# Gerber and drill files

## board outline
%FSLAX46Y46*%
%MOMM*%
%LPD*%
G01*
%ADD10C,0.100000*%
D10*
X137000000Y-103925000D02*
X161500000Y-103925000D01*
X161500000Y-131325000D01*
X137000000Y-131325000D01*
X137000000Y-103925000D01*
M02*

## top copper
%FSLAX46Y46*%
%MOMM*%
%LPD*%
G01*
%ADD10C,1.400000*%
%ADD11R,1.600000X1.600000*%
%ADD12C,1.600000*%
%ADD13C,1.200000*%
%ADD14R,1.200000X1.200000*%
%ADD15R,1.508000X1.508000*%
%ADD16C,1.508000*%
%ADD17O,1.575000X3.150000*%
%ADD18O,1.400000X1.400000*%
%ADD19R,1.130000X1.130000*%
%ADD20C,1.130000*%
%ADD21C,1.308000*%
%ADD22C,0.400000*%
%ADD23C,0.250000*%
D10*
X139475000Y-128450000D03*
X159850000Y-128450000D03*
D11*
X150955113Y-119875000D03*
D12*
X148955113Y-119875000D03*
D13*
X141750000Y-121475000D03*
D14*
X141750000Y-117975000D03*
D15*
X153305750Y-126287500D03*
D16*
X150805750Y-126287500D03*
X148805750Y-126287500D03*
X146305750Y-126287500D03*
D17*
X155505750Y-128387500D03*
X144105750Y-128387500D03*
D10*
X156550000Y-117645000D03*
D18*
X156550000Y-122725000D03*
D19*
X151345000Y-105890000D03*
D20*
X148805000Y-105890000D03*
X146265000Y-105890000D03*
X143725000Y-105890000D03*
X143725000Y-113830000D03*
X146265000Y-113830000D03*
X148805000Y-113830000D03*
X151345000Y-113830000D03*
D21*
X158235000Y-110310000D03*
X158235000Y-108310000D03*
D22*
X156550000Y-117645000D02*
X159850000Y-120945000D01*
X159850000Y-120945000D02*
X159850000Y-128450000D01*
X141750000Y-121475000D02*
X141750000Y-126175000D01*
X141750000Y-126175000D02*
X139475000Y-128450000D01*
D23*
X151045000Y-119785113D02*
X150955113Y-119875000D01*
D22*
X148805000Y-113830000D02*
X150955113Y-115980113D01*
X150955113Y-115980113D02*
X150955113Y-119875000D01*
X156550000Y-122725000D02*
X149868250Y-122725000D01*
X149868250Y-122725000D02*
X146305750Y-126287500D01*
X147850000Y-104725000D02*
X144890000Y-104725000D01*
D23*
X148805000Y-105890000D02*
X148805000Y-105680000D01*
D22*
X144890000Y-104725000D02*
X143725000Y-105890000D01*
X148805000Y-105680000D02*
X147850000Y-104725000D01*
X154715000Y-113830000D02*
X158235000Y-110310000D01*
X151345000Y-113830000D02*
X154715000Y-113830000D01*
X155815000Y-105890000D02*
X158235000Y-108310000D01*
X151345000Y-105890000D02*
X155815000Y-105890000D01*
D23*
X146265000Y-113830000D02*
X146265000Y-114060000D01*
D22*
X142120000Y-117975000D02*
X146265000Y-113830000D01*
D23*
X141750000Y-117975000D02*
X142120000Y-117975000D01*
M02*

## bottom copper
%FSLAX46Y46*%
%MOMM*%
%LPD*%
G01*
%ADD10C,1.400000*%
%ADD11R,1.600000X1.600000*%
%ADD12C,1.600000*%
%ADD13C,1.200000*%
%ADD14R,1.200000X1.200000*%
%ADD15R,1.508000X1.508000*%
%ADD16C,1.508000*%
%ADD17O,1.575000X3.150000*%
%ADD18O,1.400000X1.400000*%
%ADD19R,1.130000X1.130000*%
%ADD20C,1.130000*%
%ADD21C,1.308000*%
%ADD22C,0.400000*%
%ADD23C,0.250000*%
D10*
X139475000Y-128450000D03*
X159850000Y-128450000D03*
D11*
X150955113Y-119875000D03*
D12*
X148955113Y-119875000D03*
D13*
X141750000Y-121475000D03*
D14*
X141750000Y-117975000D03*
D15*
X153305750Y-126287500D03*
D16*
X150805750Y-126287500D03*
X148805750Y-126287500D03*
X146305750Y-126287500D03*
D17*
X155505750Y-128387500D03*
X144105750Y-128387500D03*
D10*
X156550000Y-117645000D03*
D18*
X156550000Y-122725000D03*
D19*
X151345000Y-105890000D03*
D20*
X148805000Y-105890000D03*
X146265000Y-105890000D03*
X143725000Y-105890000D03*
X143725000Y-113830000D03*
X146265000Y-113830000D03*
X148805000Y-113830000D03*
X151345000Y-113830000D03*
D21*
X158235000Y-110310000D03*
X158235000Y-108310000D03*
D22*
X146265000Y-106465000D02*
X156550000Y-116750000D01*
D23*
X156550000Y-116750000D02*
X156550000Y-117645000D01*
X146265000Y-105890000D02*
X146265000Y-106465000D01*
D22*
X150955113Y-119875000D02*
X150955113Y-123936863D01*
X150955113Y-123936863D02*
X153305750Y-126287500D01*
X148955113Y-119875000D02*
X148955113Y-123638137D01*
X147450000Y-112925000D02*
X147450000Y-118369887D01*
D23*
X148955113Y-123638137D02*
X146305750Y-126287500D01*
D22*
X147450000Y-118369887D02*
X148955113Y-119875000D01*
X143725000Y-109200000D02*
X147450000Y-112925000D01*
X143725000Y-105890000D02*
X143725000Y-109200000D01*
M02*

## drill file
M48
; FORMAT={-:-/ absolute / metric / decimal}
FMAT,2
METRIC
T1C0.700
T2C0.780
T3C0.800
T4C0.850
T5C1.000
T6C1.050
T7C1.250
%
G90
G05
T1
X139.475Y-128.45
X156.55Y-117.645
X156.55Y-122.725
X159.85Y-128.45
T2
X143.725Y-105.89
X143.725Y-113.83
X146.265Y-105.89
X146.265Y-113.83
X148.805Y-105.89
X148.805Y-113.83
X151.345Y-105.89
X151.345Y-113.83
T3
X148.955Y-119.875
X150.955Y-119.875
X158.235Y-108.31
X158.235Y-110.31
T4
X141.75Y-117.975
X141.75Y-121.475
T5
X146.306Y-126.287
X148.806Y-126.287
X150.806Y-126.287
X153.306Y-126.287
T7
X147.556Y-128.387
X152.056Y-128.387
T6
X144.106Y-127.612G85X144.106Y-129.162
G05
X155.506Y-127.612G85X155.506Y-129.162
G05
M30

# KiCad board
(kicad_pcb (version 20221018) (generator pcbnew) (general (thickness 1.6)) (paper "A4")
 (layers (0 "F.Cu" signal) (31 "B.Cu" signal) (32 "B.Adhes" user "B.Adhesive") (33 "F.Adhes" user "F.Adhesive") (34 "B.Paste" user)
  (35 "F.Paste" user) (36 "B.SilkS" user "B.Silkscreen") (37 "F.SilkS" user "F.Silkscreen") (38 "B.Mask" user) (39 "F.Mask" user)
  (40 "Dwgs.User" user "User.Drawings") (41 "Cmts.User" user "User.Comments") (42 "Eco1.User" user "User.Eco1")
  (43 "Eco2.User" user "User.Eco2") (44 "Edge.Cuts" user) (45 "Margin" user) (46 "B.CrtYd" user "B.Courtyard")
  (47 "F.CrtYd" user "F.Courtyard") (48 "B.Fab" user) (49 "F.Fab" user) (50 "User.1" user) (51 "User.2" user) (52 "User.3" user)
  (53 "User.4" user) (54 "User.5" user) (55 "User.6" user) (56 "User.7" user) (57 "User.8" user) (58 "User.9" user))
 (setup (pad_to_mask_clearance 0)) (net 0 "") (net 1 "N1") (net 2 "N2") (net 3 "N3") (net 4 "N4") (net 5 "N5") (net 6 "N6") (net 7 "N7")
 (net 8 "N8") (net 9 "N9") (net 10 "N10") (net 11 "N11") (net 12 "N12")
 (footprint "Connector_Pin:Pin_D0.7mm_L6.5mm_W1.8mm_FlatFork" (layer "F.Cu") (at 139.475 128.45)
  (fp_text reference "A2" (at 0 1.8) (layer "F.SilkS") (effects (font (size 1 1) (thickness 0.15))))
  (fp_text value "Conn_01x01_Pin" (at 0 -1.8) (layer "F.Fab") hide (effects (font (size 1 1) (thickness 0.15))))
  (pad "1" thru_hole circle (at 0 0) (size 1.4 1.4) (drill 0.7) (layers "*.Cu" "*.Mask") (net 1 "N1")))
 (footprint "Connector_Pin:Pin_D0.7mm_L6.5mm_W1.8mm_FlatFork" (layer "F.Cu") (at 159.85 128.45)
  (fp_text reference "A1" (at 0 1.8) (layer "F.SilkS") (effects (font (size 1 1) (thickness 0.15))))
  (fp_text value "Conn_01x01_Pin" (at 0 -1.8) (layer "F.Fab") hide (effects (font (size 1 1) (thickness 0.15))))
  (pad "1" thru_hole circle (at 0 0) (size 1.4 1.4) (drill 0.7) (layers "*.Cu" "*.Mask") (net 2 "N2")))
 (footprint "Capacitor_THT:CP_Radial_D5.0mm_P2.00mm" (layer "F.Cu") (at 150.955113 119.875 180)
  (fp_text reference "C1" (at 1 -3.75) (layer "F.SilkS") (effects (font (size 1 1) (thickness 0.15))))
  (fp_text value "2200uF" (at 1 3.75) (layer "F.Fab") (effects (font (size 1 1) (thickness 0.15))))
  (pad "1" thru_hole rect (at 0 0 180) (size 1.6 1.6) (drill 0.8) (layers "*.Cu" "*.Mask") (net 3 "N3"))
  (pad "2" thru_hole circle (at 2 0 180) (size 1.6 1.6) (drill 0.8) (layers "*.Cu" "*.Mask") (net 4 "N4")))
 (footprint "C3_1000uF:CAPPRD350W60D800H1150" (layer "F.Cu") (at 141.75 119.725 -90)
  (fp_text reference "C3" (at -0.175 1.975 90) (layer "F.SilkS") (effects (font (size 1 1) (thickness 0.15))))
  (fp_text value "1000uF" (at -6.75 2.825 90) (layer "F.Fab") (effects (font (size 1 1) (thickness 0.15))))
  (pad "N" thru_hole circle (at 1.75 0 270) (size 1.2 1.2) (drill 0.85) (layers "*.Cu" "*.Mask") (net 1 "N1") (solder_mask_margin 0.102))
  (pad "P" thru_hole rect (at -1.75 0 270) (size 1.2 1.2) (drill 0.85) (layers "*.Cu" "*.Mask") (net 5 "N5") (solder_mask_margin 0.102)))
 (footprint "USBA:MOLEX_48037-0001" (layer "F.Cu") (at 149.80575 128.3875)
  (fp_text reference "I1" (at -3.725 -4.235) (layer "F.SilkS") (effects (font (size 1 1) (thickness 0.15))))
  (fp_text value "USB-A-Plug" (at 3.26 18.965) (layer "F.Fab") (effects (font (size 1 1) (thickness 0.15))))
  (pad "" np_thru_hole circle (at -2.25 0) (size 1.25 1.25) (drill 1.25) (layers "*.Cu" "*.Mask"))
  (pad "" np_thru_hole circle (at 2.25 0) (size 1.25 1.25) (drill 1.25) (layers "*.Cu" "*.Mask"))
  (pad "1" thru_hole rect (at 3.5 -2.1) (size 1.508 1.508) (drill 1) (layers "*.Cu" "*.Mask") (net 3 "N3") (solder_mask_margin 0.0762))
  (pad "2" thru_hole circle (at 1 -2.1) (size 1.508 1.508) (drill 1) (layers "*.Cu" "*.Mask") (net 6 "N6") (solder_mask_margin 0.0762))
  (pad "3" thru_hole circle (at -1 -2.1) (size 1.508 1.508) (drill 1) (layers "*.Cu" "*.Mask") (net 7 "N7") (solder_mask_margin 0.0762))
  (pad "4" thru_hole circle (at -3.5 -2.1) (size 1.508 1.508) (drill 1) (layers "*.Cu" "*.Mask") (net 4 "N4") (solder_mask_margin 0.0762))
  (pad "S1" thru_hole oval (at 5.7 0) (size 1.575 3.15) (drill oval 1.05 2.6) (layers "*.Cu" "*.Mask") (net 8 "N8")
   (solder_mask_margin 0.0762))
  (pad "S2" thru_hole oval (at -5.7 0) (size 1.575 3.15) (drill oval 1.05 2.6) (layers "*.Cu" "*.Mask") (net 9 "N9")
   (solder_mask_margin 0.0762)))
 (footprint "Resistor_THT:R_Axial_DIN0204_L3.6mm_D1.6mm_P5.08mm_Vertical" (layer "F.Cu") (at 156.55 117.645 -90)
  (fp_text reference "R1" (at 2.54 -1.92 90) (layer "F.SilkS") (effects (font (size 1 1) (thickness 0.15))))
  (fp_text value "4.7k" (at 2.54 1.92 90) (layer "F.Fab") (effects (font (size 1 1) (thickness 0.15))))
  (pad "1" thru_hole circle (at 0 0 270) (size 1.4 1.4) (drill 0.7) (layers "*.Cu" "*.Mask") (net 2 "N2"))
  (pad "2" thru_hole oval (at 5.08 0 270) (size 1.4 1.4) (drill 0.7) (layers "*.Cu" "*.Mask") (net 4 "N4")))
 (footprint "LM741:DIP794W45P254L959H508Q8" (layer "F.Cu") (at 147.535 109.86 -90)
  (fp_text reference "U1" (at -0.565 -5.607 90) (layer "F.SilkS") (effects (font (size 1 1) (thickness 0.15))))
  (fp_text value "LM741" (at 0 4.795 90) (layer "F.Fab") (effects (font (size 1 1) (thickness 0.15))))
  (pad "1" thru_hole rect (at -3.97 -3.81 270) (size 1.13 1.13) (drill 0.78) (layers "*.Cu" "*.Mask") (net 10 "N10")
   (solder_mask_margin 0.102))
  (pad "2" thru_hole circle (at -3.97 -1.27 270) (size 1.13 1.13) (drill 0.78) (layers "*.Cu" "*.Mask") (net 4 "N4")
   (solder_mask_margin 0.102))
  (pad "3" thru_hole circle (at -3.97 1.27 270) (size 1.13 1.13) (drill 0.78) (layers "*.Cu" "*.Mask") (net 2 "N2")
   (solder_mask_margin 0.102))
  (pad "4" thru_hole circle (at -3.97 3.81 270) (size 1.13 1.13) (drill 0.78) (layers "*.Cu" "*.Mask") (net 4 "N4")
   (solder_mask_margin 0.102))
  (pad "5" thru_hole circle (at 3.97 3.81 270) (size 1.13 1.13) (drill 0.78) (layers "*.Cu" "*.Mask") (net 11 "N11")
   (solder_mask_margin 0.102))
  (pad "6" thru_hole circle (at 3.97 1.27 270) (size 1.13 1.13) (drill 0.78) (layers "*.Cu" "*.Mask") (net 5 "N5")
   (solder_mask_margin 0.102))
  (pad "7" thru_hole circle (at 3.97 -1.27 270) (size 1.13 1.13) (drill 0.78) (layers "*.Cu" "*.Mask") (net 3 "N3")
   (solder_mask_margin 0.102))
  (pad "8" thru_hole circle (at 3.97 -3.81 270) (size 1.13 1.13) (drill 0.78) (layers "*.Cu" "*.Mask") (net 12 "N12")
   (solder_mask_margin 0.102)))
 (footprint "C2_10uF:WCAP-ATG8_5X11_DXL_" (layer "F.Cu") (at 158.235 109.31 -90)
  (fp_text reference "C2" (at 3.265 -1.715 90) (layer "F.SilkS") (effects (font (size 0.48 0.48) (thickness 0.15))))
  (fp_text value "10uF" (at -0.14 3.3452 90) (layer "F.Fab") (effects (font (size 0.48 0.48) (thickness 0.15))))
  (pad "1" thru_hole circle (at 1 0 270) (size 1.308 1.308) (drill 0.8) (layers "*.Cu" "*.Mask") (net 12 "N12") (solder_mask_margin 0.102))
  (pad "2" thru_hole circle (at -1 0 270) (size 1.308 1.308) (drill 0.8) (layers "*.Cu" "*.Mask") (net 10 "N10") (solder_mask_margin 0.102)))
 (gr_rect (start 137 103.925) (end 161.5 131.325) (stroke (width 0.1) (type default)) (fill none) (layer "Edge.Cuts"))
 (segment (start 156.55 117.645) (end 159.85 120.945) (width 0.4) (layer "F.Cu") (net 2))
 (segment (start 159.85 120.945) (end 159.85 128.45) (width 0.4) (layer "F.Cu") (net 2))
 (segment (start 146.265 106.465) (end 156.55 116.75) (width 0.4) (layer "B.Cu") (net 2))
 (segment (start 156.55 116.75) (end 156.55 117.645) (width 0.25) (layer "B.Cu") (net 2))
 (segment (start 146.265 105.89) (end 146.265 106.465) (width 0.25) (layer "B.Cu") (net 2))
 (segment (start 141.75 121.475) (end 141.75 126.175) (width 0.4) (layer "F.Cu") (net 1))
 (segment (start 141.75 126.175) (end 139.475 128.45) (width 0.4) (layer "F.Cu") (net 1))
 (segment (start 151.045 119.785113) (end 150.955113 119.875) (width 0.25) (layer "F.Cu") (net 3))
 (segment (start 148.805 113.83) (end 150.955113 115.980113) (width 0.4) (layer "F.Cu") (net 3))
 (segment (start 150.955113 115.980113) (end 150.955113 119.875) (width 0.4) (layer "F.Cu") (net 3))
 (segment (start 150.955113 119.875) (end 150.955113 123.936863) (width 0.4) (layer "B.Cu") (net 3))
 (segment (start 150.955113 123.936863) (end 153.30575 126.2875) (width 0.4) (layer "B.Cu") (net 3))
 (segment (start 156.55 122.725) (end 149.86825 122.725) (width 0.4) (layer "F.Cu") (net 4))
 (segment (start 149.86825 122.725) (end 146.30575 126.2875) (width 0.4) (layer "F.Cu") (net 4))
 (segment (start 147.85 104.725) (end 144.89 104.725) (width 0.4) (layer "F.Cu") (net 4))
 (segment (start 148.805 105.89) (end 148.805 105.68) (width 0.25) (layer "F.Cu") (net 4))
 (segment (start 144.89 104.725) (end 143.725 105.89) (width 0.4) (layer "F.Cu") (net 4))
 (segment (start 148.805 105.68) (end 147.85 104.725) (width 0.4) (layer "F.Cu") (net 4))
 (segment (start 148.955113 119.875) (end 148.955113 123.638137) (width 0.4) (layer "B.Cu") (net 4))
 (segment (start 147.45 112.925) (end 147.45 118.369887) (width 0.4) (layer "B.Cu") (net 4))
 (segment (start 148.955113 123.638137) (end 146.30575 126.2875) (width 0.25) (layer "B.Cu") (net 4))
 (segment (start 147.45 118.369887) (end 148.955113 119.875) (width 0.4) (layer "B.Cu") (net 4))
 (segment (start 143.725 109.2) (end 147.45 112.925) (width 0.4) (layer "B.Cu") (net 4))
 (segment (start 143.725 105.89) (end 143.725 109.2) (width 0.4) (layer "B.Cu") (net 4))
 (segment (start 154.715 113.83) (end 158.235 110.31) (width 0.4) (layer "F.Cu") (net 12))
 (segment (start 151.345 113.83) (end 154.715 113.83) (width 0.4) (layer "F.Cu") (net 12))
 (segment (start 155.815 105.89) (end 158.235 108.31) (width 0.4) (layer "F.Cu") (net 10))
 (segment (start 151.345 105.89) (end 155.815 105.89) (width 0.4) (layer "F.Cu") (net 10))
 (segment (start 146.265 113.83) (end 146.265 114.06) (width 0.25) (layer "F.Cu") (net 5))
 (segment (start 142.12 117.975) (end 146.265 113.83) (width 0.4) (layer "F.Cu") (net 5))
 (segment (start 141.75 117.975) (end 142.12 117.975) (width 0.25) (layer "F.Cu") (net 5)))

